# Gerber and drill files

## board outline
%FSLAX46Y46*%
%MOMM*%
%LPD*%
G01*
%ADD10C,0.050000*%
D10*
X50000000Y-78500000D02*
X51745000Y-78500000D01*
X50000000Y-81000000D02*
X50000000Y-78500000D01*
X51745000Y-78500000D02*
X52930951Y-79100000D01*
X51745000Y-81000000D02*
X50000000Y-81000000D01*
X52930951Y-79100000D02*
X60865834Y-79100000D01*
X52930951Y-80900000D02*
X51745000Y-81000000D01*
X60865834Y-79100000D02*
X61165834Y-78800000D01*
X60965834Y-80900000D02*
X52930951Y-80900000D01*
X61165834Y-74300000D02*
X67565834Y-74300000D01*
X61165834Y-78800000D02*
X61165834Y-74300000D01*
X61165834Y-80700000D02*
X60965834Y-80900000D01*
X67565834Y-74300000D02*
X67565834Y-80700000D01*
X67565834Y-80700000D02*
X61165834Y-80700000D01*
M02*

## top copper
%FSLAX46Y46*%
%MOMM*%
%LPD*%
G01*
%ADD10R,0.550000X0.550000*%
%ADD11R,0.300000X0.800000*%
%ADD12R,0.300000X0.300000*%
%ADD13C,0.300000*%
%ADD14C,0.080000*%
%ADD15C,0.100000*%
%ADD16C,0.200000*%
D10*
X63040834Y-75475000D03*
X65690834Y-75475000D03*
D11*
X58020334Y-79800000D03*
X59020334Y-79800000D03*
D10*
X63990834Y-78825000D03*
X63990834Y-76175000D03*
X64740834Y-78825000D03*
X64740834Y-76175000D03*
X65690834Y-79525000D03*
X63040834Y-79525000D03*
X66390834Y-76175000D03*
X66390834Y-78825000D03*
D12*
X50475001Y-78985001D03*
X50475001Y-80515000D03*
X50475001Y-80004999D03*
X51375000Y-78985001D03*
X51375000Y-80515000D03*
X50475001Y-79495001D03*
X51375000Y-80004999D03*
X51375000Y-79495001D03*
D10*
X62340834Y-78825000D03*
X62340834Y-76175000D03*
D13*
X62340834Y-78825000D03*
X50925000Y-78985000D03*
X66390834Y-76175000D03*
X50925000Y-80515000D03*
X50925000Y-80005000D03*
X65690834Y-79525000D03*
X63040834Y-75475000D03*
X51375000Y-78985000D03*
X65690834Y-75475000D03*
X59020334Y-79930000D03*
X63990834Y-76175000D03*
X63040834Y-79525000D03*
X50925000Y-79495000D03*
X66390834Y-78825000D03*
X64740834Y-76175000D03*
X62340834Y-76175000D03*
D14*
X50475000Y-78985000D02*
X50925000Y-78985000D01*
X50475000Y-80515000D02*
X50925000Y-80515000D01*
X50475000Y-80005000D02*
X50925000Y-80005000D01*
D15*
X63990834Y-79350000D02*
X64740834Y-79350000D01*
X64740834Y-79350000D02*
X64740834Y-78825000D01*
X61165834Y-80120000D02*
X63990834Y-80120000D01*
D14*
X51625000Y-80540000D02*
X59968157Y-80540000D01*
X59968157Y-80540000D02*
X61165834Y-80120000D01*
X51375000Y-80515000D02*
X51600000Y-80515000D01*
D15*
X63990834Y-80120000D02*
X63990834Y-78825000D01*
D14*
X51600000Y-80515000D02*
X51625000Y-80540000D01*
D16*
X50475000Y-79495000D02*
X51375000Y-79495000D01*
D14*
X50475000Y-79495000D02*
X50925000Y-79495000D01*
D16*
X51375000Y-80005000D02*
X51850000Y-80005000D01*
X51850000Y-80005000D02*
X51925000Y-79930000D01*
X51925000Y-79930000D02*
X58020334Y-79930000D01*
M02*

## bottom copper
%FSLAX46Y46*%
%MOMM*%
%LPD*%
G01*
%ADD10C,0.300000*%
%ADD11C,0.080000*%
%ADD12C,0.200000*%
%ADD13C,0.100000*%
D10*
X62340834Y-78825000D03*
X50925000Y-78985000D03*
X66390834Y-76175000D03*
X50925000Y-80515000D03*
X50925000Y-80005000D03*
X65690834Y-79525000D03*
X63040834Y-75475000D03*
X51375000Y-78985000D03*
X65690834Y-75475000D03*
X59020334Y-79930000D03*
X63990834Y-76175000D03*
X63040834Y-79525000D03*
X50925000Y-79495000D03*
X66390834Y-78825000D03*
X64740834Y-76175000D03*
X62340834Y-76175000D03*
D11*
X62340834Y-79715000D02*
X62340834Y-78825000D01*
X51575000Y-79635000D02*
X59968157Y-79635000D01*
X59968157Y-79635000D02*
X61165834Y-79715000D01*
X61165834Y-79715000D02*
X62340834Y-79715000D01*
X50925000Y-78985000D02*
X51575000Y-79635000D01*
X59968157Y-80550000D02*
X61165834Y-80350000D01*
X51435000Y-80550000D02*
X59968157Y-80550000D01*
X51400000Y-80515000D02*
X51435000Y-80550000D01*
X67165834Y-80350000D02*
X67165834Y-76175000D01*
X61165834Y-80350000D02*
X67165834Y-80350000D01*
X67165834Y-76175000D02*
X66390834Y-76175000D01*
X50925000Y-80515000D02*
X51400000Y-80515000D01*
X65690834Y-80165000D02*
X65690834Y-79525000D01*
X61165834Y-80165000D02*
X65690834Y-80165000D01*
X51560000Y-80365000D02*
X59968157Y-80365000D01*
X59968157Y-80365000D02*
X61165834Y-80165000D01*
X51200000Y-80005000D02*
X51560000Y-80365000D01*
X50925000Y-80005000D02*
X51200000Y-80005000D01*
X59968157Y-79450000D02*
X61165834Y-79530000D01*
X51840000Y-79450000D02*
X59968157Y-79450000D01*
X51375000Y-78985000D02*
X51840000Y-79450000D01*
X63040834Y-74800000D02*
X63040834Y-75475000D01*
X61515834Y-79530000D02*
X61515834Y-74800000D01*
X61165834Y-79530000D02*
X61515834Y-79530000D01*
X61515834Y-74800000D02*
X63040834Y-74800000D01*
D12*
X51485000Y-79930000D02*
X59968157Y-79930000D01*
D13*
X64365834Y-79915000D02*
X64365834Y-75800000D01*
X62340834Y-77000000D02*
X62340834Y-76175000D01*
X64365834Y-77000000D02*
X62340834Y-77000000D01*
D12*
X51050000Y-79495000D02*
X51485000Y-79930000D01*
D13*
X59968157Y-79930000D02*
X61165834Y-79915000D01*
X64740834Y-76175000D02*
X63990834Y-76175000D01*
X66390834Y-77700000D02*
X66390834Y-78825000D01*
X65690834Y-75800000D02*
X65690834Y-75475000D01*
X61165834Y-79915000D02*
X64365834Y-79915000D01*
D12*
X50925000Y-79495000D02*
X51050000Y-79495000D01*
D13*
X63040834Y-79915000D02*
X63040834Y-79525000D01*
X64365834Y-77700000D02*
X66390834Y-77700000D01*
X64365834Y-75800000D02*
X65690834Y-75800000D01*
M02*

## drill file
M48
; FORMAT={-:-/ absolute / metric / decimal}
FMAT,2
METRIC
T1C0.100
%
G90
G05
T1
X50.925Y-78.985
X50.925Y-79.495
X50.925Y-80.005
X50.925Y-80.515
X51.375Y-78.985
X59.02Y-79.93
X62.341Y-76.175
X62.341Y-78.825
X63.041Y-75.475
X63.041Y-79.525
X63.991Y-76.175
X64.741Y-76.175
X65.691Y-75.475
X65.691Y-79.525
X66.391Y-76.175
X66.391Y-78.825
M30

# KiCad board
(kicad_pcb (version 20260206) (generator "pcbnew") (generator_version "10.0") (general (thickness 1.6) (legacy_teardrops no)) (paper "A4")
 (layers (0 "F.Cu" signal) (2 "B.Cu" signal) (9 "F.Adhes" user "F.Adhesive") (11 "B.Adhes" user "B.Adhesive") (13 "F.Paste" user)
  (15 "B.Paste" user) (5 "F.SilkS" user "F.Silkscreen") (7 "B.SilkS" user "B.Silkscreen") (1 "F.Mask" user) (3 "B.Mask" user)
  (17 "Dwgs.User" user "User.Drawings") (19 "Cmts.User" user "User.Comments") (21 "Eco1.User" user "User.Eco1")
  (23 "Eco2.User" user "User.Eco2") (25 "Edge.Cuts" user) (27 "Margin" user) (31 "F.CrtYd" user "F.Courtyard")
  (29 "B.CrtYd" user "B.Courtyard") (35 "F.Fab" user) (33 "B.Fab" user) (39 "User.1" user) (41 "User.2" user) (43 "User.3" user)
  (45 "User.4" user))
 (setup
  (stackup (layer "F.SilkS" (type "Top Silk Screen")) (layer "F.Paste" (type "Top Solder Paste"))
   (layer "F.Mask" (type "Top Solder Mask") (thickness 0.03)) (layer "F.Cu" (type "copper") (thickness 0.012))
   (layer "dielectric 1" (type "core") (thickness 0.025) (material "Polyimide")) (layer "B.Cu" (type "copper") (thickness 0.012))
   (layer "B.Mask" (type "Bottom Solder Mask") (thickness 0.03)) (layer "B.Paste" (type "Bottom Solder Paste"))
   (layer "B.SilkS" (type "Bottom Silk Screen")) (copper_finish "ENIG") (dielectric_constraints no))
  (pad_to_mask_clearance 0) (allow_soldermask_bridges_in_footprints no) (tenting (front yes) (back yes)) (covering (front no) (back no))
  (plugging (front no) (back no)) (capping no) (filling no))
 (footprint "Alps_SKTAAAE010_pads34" (layer "F.Cu") (at 66.765834 77.5 -90)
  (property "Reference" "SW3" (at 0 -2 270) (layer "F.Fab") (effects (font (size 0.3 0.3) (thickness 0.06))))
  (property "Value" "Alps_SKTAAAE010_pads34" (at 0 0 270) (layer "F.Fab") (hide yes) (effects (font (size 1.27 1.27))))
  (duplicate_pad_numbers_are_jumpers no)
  (pad "3" smd rect (at -1.325 0.375 270) (size 0.55 0.55) (layers "F.Cu" "F.Mask" "F.Paste") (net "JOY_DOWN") (solder_mask_margin 0.05)
   (thermal_bridge_angle 45))
  (pad "4" smd rect (at 1.325 0.375 270) (size 0.55 0.55) (layers "F.Cu" "F.Mask" "F.Paste") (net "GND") (solder_mask_margin 0.05)
   (thermal_bridge_angle 45)))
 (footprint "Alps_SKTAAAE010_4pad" (layer "F.Cu") (at 64.365834 77.5 90)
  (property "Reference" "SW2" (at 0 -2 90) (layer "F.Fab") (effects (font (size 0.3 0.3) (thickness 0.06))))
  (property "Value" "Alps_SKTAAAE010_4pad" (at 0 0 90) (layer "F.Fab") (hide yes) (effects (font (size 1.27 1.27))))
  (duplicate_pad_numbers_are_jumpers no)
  (pad "1" smd rect (at -1.325 -0.375 90) (size 0.55 0.55) (layers "F.Cu" "F.Mask" "F.Paste") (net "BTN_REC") (solder_mask_margin 0.05)
   (thermal_bridge_angle 45))
  (pad "2" smd rect (at 1.325 -0.375 90) (size 0.55 0.55) (layers "F.Cu" "F.Mask" "F.Paste") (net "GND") (solder_mask_margin 0.05)
   (thermal_bridge_angle 45))
  (pad "3" smd rect (at -1.325 0.375 90) (size 0.55 0.55) (layers "F.Cu" "F.Mask" "F.Paste") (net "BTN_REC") (solder_mask_margin 0.05)
   (thermal_bridge_angle 45))
  (pad "4" smd rect (at 1.325 0.375 90) (size 0.55 0.55) (layers "F.Cu" "F.Mask" "F.Paste") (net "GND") (solder_mask_margin 0.05)
   (thermal_bridge_angle 45)))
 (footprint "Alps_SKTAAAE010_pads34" (layer "F.Cu") (at 64.365834 79.9 180)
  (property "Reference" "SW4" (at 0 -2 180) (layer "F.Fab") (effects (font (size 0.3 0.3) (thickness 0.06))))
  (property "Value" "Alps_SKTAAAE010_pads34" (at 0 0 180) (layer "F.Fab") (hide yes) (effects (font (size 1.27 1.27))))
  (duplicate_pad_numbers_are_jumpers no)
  (pad "3" smd rect (at -1.325 0.375 180) (size 0.55 0.55) (layers "F.Cu" "F.Mask" "F.Paste") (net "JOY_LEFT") (solder_mask_margin 0.05)
   (thermal_bridge_angle 45))
  (pad "4" smd rect (at 1.325 0.375 180) (size 0.55 0.55) (layers "F.Cu" "F.Mask" "F.Paste") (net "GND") (solder_mask_margin 0.05)
   (thermal_bridge_angle 45)))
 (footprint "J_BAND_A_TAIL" (layer "F.Cu") (at 50.9 79.75)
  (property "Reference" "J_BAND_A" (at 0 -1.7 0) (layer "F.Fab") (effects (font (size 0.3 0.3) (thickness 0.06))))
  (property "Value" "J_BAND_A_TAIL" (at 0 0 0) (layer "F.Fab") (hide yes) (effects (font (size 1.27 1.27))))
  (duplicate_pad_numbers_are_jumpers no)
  (pad "1" smd rect (at -0.424999 -0.764999) (size 0.3 0.3) (layers "F.Cu" "F.Mask") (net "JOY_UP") (solder_mask_margin 0.05)
   (thermal_bridge_angle 45))
  (pad "2" smd rect (at -0.424999 0.765) (size 0.3 0.3) (layers "F.Cu" "F.Mask") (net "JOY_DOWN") (solder_mask_margin 0.05)
   (thermal_bridge_angle 45))
  (pad "3" smd rect (at -0.424999 0.254999) (size 0.3 0.3) (layers "F.Cu" "F.Mask") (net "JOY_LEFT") (solder_mask_margin 0.05)
   (thermal_bridge_angle 45))
  (pad "4" smd rect (at 0.475 -0.764999) (size 0.3 0.3) (layers "F.Cu" "F.Mask") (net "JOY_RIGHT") (solder_mask_margin 0.05)
   (thermal_bridge_angle 45))
  (pad "5" smd rect (at 0.475 0.765) (size 0.3 0.3) (layers "F.Cu" "F.Mask") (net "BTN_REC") (solder_mask_margin 0.05)
   (thermal_bridge_angle 45))
  (pad "6" smd rect (at -0.424999 -0.254999) (size 0.3 0.3) (layers "F.Cu" "F.Mask") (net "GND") (solder_mask_margin 0.05)
   (thermal_bridge_angle 45))
  (pad "7" smd rect (at 0.475 0.254999) (size 0.3 0.3) (layers "F.Cu" "F.Mask") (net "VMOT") (solder_mask_margin 0.05)
   (thermal_bridge_angle 45))
  (pad "8" smd rect (at 0.475 -0.254999) (size 0.3 0.3) (layers "F.Cu" "F.Mask") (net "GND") (solder_mask_margin 0.05)
   (thermal_bridge_angle 45)))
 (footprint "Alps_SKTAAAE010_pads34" (layer "F.Cu") (at 61.965834 77.5 90)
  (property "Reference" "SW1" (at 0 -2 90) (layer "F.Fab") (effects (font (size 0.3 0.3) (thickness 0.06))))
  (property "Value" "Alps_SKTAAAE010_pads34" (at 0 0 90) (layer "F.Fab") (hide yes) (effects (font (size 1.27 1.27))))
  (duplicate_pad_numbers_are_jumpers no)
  (pad "3" smd rect (at -1.325 0.375 90) (size 0.55 0.55) (layers "F.Cu" "F.Mask" "F.Paste") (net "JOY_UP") (solder_mask_margin 0.05)
   (thermal_bridge_angle 45))
  (pad "4" smd rect (at 1.325 0.375 90) (size 0.55 0.55) (layers "F.Cu" "F.Mask" "F.Paste") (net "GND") (solder_mask_margin 0.05)
   (thermal_bridge_angle 45)))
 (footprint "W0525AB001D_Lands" (layer "F.Cu") (at 58.520334 79.93)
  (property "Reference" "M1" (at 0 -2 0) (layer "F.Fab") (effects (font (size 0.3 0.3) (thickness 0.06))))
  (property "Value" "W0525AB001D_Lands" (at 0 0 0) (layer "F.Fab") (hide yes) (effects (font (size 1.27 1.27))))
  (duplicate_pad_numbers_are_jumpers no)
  (pad "1" smd rect (at -0.5 -0.13) (size 0.3 0.8) (layers "F.Cu" "F.Mask") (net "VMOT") (solder_mask_margin 0.05) (thermal_bridge_angle 45))
  (pad "2" smd rect (at 0.5 -0.13) (size 0.3 0.8) (layers "F.Cu" "F.Mask") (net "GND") (solder_mask_margin 0.05) (thermal_bridge_angle 45)))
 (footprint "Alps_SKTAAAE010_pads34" (layer "F.Cu") (at 64.365834 75.1)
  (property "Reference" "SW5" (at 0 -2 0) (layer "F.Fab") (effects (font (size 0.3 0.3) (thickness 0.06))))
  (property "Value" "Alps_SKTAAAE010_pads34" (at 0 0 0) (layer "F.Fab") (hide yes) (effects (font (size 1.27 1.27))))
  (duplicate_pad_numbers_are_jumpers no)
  (pad "3" smd rect (at -1.325 0.375) (size 0.55 0.55) (layers "F.Cu" "F.Mask" "F.Paste") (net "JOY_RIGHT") (solder_mask_margin 0.05)
   (thermal_bridge_angle 45))
  (pad "4" smd rect (at 1.325 0.375) (size 0.55 0.55) (layers "F.Cu" "F.Mask" "F.Paste") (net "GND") (solder_mask_margin 0.05)
   (thermal_bridge_angle 45)))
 (gr_line (start 50 78.5) (end 51.745 78.5) (stroke (width 0.05) (type default)) (layer "Edge.Cuts"))
 (gr_line (start 50 81) (end 50 78.5) (stroke (width 0.05) (type default)) (layer "Edge.Cuts"))
 (gr_line (start 51.745 78.5) (end 52.930951 79.1) (stroke (width 0.05) (type default)) (layer "Edge.Cuts"))
 (gr_line (start 51.745 81) (end 50 81) (stroke (width 0.05) (type default)) (layer "Edge.Cuts"))
 (gr_line (start 52.930951 79.1) (end 60.865834 79.1) (stroke (width 0.05) (type default)) (layer "Edge.Cuts"))
 (gr_line (start 52.930951 80.9) (end 51.745 81) (stroke (width 0.05) (type default)) (layer "Edge.Cuts"))
 (gr_line (start 60.865834 79.1) (end 61.165834 78.8) (stroke (width 0.05) (type default)) (layer "Edge.Cuts"))
 (gr_line (start 60.965834 80.9) (end 52.930951 80.9) (stroke (width 0.05) (type default)) (layer "Edge.Cuts"))
 (gr_line (start 61.165834 74.3) (end 67.565834 74.3) (stroke (width 0.05) (type default)) (layer "Edge.Cuts"))
 (gr_line (start 61.165834 78.8) (end 61.165834 74.3) (stroke (width 0.05) (type default)) (layer "Edge.Cuts"))
 (gr_line (start 61.165834 80.7) (end 60.965834 80.9) (stroke (width 0.05) (type default)) (layer "Edge.Cuts"))
 (gr_line (start 67.565834 74.3) (end 67.565834 80.7) (stroke (width 0.05) (type default)) (layer "Edge.Cuts"))
 (gr_line (start 67.565834 80.7) (end 61.165834 80.7) (stroke (width 0.05) (type default)) (layer "Edge.Cuts"))
 (segment (start 50.475 78.985) (end 50.925 78.985) (width 0.08) (layer "F.Cu") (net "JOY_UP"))
 (via (at 62.340834 78.825) (size 0.3) (drill 0.1) (layers "F.Cu" "B.Cu") (tenting (front yes) (back yes)) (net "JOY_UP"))
 (via (at 50.925 78.985) (size 0.3) (drill 0.1) (layers "F.Cu" "B.Cu") (tenting (front yes) (back yes)) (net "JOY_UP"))
 (segment (start 62.340834 79.715) (end 62.340834 78.825) (width 0.08) (layer "B.Cu") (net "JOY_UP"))
 (segment (start 51.575 79.635) (end 59.968157 79.635) (width 0.08) (layer "B.Cu") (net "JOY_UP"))
 (segment (start 50.925 78.985) (end 51.575 79.635) (width 0.08) (layer "B.Cu") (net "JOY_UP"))
 (segment (start 59.968157 79.635) (end 61.165834 79.715) (width 0.08) (layer "B.Cu") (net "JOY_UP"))
 (segment (start 61.165834 79.715) (end 62.340834 79.715) (width 0.08) (layer "B.Cu") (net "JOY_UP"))
 (segment (start 50.475 80.515) (end 50.925 80.515) (width 0.08) (layer "F.Cu") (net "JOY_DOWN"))
 (via (at 66.390834 76.175) (size 0.3) (drill 0.1) (layers "F.Cu" "B.Cu") (tenting (front yes) (back yes)) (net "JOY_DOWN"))
 (via (at 50.925 80.515) (size 0.3) (drill 0.1) (layers "F.Cu" "B.Cu") (tenting (front yes) (back yes)) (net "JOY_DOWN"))
 (segment (start 50.925 80.515) (end 51.4 80.515) (width 0.08) (layer "B.Cu") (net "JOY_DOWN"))
 (segment (start 59.968157 80.55) (end 61.165834 80.35) (width 0.08) (layer "B.Cu") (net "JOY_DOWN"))
 (segment (start 61.165834 80.35) (end 67.165834 80.35) (width 0.08) (layer "B.Cu") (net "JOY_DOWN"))
 (segment (start 67.165834 76.175) (end 66.390834 76.175) (width 0.08) (layer "B.Cu") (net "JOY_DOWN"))
 (segment (start 51.435 80.55) (end 59.968157 80.55) (width 0.08) (layer "B.Cu") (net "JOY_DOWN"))
 (segment (start 67.165834 80.35) (end 67.165834 76.175) (width 0.08) (layer "B.Cu") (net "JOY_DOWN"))
 (segment (start 51.4 80.515) (end 51.435 80.55) (width 0.08) (layer "B.Cu") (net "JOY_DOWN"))
 (segment (start 50.475 80.005) (end 50.925 80.005) (width 0.08) (layer "F.Cu") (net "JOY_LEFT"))
 (via (at 50.925 80.005) (size 0.3) (drill 0.1) (layers "F.Cu" "B.Cu") (tenting (front yes) (back yes)) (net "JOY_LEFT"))
 (via (at 65.690834 79.525) (size 0.3) (drill 0.1) (layers "F.Cu" "B.Cu") (tenting (front yes) (back yes)) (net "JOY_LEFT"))
 (segment (start 59.968157 80.365) (end 61.165834 80.165) (width 0.08) (layer "B.Cu") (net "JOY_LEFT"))
 (segment (start 50.925 80.005) (end 51.2 80.005) (width 0.08) (layer "B.Cu") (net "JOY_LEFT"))
 (segment (start 65.690834 80.165) (end 65.690834 79.525) (width 0.08) (layer "B.Cu") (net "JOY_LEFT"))
 (segment (start 61.165834 80.165) (end 65.690834 80.165) (width 0.08) (layer "B.Cu") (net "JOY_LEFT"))
 (segment (start 51.56 80.365) (end 59.968157 80.365) (width 0.08) (layer "B.Cu") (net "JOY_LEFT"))
 (segment (start 51.2 80.005) (end 51.56 80.365) (width 0.08) (layer "B.Cu") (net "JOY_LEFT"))
 (via (at 51.375 78.985) (size 0.3) (drill 0.1) (layers "F.Cu" "B.Cu") (tenting (front yes) (back yes)) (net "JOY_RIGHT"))
 (via (at 63.040834 75.475) (size 0.3) (drill 0.1) (layers "F.Cu" "B.Cu") (tenting (front yes) (back yes)) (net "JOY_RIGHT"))
 (segment (start 61.165834 79.53) (end 61.515834 79.53) (width 0.08) (layer "B.Cu") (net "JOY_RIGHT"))
 (segment (start 51.375 78.985) (end 51.84 79.45) (width 0.08) (layer "B.Cu") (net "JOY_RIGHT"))
 (segment (start 61.515834 79.53) (end 61.515834 74.8) (width 0.08) (layer "B.Cu") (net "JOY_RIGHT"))
 (segment (start 51.84 79.45) (end 59.968157 79.45) (width 0.08) (layer "B.Cu") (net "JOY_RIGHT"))
 (segment (start 61.515834 74.8) (end 63.040834 74.8) (width 0.08) (layer "B.Cu") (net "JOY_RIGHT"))
 (segment (start 59.968157 79.45) (end 61.165834 79.53) (width 0.08) (layer "B.Cu") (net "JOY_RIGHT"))
 (segment (start 63.040834 74.8) (end 63.040834 75.475) (width 0.08) (layer "B.Cu") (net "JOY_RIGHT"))
 (segment (start 64.740834 79.35) (end 64.740834 78.825) (width 0.1) (layer "F.Cu") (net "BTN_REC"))
 (segment (start 51.6 80.515) (end 51.625 80.54) (width 0.08) (layer "F.Cu") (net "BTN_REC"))
 (segment (start 63.990834 80.12) (end 63.990834 78.825) (width 0.1) (layer "F.Cu") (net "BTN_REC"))
 (segment (start 51.625 80.54) (end 59.968157 80.54) (width 0.08) (layer "F.Cu") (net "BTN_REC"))
 (segment (start 59.968157 80.54) (end 61.165834 80.12) (width 0.08) (layer "F.Cu") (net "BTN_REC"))
 (segment (start 63.990834 79.35) (end 64.740834 79.35) (width 0.1) (layer "F.Cu") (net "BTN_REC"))
 (segment (start 51.375 80.515) (end 51.6 80.515) (width 0.08) (layer "F.Cu") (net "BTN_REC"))
 (segment (start 61.165834 80.12) (end 63.990834 80.12) (width 0.1) (layer "F.Cu") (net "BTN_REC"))
 (segment (start 50.475 79.495) (end 51.375 79.495) (width 0.2) (layer "F.Cu") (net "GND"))
 (segment (start 50.475 79.495) (end 50.925 79.495) (width 0.08) (layer "F.Cu") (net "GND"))
 (via (at 63.990834 76.175) (size 0.3) (drill 0.1) (layers "F.Cu" "B.Cu") (tenting (front yes) (back yes)) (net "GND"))
 (via (at 66.390834 78.825) (size 0.3) (drill 0.1) (layers "F.Cu" "B.Cu") (tenting (front yes) (back yes)) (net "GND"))
 (via (at 63.040834 79.525) (size 0.3) (drill 0.1) (layers "F.Cu" "B.Cu") (tenting (front yes) (back yes)) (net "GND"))
 (via (at 62.340834 76.175) (size 0.3) (drill 0.1) (layers "F.Cu" "B.Cu") (tenting (front yes) (back yes)) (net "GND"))
 (via (at 50.925 79.495) (size 0.3) (drill 0.1) (layers "F.Cu" "B.Cu") (tenting (front yes) (back yes)) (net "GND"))
 (via (at 64.740834 76.175) (size 0.3) (drill 0.1) (layers "F.Cu" "B.Cu") (tenting (front yes) (back yes)) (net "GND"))
 (via (at 65.690834 75.475) (size 0.3) (drill 0.1) (layers "F.Cu" "B.Cu") (tenting (front yes) (back yes)) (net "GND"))
 (via (at 59.020334 79.93) (size 0.3) (drill 0.1) (layers "F.Cu" "B.Cu") (tenting (front yes) (back yes)) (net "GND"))
 (segment (start 59.968157 79.93) (end 61.165834 79.915) (width 0.1) (layer "B.Cu") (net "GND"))
 (segment (start 61.165834 79.915) (end 64.365834 79.915) (width 0.1) (layer "B.Cu") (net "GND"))
 (segment (start 65.690834 75.8) (end 65.690834 75.475) (width 0.1) (layer "B.Cu") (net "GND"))
 (segment (start 64.740834 76.175) (end 63.990834 76.175) (width 0.1) (layer "B.Cu") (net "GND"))
 (segment (start 63.040834 79.915) (end 63.040834 79.525) (width 0.1) (layer "B.Cu") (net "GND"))
 (segment (start 51.485 79.93) (end 59.968157 79.93) (width 0.2) (layer "B.Cu") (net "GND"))
 (segment (start 64.365834 75.8) (end 65.690834 75.8) (width 0.1) (layer "B.Cu") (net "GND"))
 (segment (start 64.365834 79.915) (end 64.365834 75.8) (width 0.1) (layer "B.Cu") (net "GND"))
 (segment (start 66.390834 77.7) (end 66.390834 78.825) (width 0.1) (layer "B.Cu") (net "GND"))
 (segment (start 64.365834 77.7) (end 66.390834 77.7) (width 0.1) (layer "B.Cu") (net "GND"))
 (segment (start 50.925 79.495) (end 51.05 79.495) (width 0.2) (layer "B.Cu") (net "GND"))
 (segment (start 51.05 79.495) (end 51.485 79.93) (width 0.2) (layer "B.Cu") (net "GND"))
 (segment (start 64.365834 77) (end 62.340834 77) (width 0.1) (layer "B.Cu") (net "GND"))
 (segment (start 62.340834 77) (end 62.340834 76.175) (width 0.1) (layer "B.Cu") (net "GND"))
 (segment (start 51.85 80.005) (end 51.925 79.93) (width 0.2) (layer "F.Cu") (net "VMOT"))
 (segment (start 51.925 79.93) (end 58.020334 79.93) (width 0.2) (layer "F.Cu") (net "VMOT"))
 (segment (start 51.375 80.005) (end 51.85 80.005) (width 0.2) (layer "F.Cu") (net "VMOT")))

